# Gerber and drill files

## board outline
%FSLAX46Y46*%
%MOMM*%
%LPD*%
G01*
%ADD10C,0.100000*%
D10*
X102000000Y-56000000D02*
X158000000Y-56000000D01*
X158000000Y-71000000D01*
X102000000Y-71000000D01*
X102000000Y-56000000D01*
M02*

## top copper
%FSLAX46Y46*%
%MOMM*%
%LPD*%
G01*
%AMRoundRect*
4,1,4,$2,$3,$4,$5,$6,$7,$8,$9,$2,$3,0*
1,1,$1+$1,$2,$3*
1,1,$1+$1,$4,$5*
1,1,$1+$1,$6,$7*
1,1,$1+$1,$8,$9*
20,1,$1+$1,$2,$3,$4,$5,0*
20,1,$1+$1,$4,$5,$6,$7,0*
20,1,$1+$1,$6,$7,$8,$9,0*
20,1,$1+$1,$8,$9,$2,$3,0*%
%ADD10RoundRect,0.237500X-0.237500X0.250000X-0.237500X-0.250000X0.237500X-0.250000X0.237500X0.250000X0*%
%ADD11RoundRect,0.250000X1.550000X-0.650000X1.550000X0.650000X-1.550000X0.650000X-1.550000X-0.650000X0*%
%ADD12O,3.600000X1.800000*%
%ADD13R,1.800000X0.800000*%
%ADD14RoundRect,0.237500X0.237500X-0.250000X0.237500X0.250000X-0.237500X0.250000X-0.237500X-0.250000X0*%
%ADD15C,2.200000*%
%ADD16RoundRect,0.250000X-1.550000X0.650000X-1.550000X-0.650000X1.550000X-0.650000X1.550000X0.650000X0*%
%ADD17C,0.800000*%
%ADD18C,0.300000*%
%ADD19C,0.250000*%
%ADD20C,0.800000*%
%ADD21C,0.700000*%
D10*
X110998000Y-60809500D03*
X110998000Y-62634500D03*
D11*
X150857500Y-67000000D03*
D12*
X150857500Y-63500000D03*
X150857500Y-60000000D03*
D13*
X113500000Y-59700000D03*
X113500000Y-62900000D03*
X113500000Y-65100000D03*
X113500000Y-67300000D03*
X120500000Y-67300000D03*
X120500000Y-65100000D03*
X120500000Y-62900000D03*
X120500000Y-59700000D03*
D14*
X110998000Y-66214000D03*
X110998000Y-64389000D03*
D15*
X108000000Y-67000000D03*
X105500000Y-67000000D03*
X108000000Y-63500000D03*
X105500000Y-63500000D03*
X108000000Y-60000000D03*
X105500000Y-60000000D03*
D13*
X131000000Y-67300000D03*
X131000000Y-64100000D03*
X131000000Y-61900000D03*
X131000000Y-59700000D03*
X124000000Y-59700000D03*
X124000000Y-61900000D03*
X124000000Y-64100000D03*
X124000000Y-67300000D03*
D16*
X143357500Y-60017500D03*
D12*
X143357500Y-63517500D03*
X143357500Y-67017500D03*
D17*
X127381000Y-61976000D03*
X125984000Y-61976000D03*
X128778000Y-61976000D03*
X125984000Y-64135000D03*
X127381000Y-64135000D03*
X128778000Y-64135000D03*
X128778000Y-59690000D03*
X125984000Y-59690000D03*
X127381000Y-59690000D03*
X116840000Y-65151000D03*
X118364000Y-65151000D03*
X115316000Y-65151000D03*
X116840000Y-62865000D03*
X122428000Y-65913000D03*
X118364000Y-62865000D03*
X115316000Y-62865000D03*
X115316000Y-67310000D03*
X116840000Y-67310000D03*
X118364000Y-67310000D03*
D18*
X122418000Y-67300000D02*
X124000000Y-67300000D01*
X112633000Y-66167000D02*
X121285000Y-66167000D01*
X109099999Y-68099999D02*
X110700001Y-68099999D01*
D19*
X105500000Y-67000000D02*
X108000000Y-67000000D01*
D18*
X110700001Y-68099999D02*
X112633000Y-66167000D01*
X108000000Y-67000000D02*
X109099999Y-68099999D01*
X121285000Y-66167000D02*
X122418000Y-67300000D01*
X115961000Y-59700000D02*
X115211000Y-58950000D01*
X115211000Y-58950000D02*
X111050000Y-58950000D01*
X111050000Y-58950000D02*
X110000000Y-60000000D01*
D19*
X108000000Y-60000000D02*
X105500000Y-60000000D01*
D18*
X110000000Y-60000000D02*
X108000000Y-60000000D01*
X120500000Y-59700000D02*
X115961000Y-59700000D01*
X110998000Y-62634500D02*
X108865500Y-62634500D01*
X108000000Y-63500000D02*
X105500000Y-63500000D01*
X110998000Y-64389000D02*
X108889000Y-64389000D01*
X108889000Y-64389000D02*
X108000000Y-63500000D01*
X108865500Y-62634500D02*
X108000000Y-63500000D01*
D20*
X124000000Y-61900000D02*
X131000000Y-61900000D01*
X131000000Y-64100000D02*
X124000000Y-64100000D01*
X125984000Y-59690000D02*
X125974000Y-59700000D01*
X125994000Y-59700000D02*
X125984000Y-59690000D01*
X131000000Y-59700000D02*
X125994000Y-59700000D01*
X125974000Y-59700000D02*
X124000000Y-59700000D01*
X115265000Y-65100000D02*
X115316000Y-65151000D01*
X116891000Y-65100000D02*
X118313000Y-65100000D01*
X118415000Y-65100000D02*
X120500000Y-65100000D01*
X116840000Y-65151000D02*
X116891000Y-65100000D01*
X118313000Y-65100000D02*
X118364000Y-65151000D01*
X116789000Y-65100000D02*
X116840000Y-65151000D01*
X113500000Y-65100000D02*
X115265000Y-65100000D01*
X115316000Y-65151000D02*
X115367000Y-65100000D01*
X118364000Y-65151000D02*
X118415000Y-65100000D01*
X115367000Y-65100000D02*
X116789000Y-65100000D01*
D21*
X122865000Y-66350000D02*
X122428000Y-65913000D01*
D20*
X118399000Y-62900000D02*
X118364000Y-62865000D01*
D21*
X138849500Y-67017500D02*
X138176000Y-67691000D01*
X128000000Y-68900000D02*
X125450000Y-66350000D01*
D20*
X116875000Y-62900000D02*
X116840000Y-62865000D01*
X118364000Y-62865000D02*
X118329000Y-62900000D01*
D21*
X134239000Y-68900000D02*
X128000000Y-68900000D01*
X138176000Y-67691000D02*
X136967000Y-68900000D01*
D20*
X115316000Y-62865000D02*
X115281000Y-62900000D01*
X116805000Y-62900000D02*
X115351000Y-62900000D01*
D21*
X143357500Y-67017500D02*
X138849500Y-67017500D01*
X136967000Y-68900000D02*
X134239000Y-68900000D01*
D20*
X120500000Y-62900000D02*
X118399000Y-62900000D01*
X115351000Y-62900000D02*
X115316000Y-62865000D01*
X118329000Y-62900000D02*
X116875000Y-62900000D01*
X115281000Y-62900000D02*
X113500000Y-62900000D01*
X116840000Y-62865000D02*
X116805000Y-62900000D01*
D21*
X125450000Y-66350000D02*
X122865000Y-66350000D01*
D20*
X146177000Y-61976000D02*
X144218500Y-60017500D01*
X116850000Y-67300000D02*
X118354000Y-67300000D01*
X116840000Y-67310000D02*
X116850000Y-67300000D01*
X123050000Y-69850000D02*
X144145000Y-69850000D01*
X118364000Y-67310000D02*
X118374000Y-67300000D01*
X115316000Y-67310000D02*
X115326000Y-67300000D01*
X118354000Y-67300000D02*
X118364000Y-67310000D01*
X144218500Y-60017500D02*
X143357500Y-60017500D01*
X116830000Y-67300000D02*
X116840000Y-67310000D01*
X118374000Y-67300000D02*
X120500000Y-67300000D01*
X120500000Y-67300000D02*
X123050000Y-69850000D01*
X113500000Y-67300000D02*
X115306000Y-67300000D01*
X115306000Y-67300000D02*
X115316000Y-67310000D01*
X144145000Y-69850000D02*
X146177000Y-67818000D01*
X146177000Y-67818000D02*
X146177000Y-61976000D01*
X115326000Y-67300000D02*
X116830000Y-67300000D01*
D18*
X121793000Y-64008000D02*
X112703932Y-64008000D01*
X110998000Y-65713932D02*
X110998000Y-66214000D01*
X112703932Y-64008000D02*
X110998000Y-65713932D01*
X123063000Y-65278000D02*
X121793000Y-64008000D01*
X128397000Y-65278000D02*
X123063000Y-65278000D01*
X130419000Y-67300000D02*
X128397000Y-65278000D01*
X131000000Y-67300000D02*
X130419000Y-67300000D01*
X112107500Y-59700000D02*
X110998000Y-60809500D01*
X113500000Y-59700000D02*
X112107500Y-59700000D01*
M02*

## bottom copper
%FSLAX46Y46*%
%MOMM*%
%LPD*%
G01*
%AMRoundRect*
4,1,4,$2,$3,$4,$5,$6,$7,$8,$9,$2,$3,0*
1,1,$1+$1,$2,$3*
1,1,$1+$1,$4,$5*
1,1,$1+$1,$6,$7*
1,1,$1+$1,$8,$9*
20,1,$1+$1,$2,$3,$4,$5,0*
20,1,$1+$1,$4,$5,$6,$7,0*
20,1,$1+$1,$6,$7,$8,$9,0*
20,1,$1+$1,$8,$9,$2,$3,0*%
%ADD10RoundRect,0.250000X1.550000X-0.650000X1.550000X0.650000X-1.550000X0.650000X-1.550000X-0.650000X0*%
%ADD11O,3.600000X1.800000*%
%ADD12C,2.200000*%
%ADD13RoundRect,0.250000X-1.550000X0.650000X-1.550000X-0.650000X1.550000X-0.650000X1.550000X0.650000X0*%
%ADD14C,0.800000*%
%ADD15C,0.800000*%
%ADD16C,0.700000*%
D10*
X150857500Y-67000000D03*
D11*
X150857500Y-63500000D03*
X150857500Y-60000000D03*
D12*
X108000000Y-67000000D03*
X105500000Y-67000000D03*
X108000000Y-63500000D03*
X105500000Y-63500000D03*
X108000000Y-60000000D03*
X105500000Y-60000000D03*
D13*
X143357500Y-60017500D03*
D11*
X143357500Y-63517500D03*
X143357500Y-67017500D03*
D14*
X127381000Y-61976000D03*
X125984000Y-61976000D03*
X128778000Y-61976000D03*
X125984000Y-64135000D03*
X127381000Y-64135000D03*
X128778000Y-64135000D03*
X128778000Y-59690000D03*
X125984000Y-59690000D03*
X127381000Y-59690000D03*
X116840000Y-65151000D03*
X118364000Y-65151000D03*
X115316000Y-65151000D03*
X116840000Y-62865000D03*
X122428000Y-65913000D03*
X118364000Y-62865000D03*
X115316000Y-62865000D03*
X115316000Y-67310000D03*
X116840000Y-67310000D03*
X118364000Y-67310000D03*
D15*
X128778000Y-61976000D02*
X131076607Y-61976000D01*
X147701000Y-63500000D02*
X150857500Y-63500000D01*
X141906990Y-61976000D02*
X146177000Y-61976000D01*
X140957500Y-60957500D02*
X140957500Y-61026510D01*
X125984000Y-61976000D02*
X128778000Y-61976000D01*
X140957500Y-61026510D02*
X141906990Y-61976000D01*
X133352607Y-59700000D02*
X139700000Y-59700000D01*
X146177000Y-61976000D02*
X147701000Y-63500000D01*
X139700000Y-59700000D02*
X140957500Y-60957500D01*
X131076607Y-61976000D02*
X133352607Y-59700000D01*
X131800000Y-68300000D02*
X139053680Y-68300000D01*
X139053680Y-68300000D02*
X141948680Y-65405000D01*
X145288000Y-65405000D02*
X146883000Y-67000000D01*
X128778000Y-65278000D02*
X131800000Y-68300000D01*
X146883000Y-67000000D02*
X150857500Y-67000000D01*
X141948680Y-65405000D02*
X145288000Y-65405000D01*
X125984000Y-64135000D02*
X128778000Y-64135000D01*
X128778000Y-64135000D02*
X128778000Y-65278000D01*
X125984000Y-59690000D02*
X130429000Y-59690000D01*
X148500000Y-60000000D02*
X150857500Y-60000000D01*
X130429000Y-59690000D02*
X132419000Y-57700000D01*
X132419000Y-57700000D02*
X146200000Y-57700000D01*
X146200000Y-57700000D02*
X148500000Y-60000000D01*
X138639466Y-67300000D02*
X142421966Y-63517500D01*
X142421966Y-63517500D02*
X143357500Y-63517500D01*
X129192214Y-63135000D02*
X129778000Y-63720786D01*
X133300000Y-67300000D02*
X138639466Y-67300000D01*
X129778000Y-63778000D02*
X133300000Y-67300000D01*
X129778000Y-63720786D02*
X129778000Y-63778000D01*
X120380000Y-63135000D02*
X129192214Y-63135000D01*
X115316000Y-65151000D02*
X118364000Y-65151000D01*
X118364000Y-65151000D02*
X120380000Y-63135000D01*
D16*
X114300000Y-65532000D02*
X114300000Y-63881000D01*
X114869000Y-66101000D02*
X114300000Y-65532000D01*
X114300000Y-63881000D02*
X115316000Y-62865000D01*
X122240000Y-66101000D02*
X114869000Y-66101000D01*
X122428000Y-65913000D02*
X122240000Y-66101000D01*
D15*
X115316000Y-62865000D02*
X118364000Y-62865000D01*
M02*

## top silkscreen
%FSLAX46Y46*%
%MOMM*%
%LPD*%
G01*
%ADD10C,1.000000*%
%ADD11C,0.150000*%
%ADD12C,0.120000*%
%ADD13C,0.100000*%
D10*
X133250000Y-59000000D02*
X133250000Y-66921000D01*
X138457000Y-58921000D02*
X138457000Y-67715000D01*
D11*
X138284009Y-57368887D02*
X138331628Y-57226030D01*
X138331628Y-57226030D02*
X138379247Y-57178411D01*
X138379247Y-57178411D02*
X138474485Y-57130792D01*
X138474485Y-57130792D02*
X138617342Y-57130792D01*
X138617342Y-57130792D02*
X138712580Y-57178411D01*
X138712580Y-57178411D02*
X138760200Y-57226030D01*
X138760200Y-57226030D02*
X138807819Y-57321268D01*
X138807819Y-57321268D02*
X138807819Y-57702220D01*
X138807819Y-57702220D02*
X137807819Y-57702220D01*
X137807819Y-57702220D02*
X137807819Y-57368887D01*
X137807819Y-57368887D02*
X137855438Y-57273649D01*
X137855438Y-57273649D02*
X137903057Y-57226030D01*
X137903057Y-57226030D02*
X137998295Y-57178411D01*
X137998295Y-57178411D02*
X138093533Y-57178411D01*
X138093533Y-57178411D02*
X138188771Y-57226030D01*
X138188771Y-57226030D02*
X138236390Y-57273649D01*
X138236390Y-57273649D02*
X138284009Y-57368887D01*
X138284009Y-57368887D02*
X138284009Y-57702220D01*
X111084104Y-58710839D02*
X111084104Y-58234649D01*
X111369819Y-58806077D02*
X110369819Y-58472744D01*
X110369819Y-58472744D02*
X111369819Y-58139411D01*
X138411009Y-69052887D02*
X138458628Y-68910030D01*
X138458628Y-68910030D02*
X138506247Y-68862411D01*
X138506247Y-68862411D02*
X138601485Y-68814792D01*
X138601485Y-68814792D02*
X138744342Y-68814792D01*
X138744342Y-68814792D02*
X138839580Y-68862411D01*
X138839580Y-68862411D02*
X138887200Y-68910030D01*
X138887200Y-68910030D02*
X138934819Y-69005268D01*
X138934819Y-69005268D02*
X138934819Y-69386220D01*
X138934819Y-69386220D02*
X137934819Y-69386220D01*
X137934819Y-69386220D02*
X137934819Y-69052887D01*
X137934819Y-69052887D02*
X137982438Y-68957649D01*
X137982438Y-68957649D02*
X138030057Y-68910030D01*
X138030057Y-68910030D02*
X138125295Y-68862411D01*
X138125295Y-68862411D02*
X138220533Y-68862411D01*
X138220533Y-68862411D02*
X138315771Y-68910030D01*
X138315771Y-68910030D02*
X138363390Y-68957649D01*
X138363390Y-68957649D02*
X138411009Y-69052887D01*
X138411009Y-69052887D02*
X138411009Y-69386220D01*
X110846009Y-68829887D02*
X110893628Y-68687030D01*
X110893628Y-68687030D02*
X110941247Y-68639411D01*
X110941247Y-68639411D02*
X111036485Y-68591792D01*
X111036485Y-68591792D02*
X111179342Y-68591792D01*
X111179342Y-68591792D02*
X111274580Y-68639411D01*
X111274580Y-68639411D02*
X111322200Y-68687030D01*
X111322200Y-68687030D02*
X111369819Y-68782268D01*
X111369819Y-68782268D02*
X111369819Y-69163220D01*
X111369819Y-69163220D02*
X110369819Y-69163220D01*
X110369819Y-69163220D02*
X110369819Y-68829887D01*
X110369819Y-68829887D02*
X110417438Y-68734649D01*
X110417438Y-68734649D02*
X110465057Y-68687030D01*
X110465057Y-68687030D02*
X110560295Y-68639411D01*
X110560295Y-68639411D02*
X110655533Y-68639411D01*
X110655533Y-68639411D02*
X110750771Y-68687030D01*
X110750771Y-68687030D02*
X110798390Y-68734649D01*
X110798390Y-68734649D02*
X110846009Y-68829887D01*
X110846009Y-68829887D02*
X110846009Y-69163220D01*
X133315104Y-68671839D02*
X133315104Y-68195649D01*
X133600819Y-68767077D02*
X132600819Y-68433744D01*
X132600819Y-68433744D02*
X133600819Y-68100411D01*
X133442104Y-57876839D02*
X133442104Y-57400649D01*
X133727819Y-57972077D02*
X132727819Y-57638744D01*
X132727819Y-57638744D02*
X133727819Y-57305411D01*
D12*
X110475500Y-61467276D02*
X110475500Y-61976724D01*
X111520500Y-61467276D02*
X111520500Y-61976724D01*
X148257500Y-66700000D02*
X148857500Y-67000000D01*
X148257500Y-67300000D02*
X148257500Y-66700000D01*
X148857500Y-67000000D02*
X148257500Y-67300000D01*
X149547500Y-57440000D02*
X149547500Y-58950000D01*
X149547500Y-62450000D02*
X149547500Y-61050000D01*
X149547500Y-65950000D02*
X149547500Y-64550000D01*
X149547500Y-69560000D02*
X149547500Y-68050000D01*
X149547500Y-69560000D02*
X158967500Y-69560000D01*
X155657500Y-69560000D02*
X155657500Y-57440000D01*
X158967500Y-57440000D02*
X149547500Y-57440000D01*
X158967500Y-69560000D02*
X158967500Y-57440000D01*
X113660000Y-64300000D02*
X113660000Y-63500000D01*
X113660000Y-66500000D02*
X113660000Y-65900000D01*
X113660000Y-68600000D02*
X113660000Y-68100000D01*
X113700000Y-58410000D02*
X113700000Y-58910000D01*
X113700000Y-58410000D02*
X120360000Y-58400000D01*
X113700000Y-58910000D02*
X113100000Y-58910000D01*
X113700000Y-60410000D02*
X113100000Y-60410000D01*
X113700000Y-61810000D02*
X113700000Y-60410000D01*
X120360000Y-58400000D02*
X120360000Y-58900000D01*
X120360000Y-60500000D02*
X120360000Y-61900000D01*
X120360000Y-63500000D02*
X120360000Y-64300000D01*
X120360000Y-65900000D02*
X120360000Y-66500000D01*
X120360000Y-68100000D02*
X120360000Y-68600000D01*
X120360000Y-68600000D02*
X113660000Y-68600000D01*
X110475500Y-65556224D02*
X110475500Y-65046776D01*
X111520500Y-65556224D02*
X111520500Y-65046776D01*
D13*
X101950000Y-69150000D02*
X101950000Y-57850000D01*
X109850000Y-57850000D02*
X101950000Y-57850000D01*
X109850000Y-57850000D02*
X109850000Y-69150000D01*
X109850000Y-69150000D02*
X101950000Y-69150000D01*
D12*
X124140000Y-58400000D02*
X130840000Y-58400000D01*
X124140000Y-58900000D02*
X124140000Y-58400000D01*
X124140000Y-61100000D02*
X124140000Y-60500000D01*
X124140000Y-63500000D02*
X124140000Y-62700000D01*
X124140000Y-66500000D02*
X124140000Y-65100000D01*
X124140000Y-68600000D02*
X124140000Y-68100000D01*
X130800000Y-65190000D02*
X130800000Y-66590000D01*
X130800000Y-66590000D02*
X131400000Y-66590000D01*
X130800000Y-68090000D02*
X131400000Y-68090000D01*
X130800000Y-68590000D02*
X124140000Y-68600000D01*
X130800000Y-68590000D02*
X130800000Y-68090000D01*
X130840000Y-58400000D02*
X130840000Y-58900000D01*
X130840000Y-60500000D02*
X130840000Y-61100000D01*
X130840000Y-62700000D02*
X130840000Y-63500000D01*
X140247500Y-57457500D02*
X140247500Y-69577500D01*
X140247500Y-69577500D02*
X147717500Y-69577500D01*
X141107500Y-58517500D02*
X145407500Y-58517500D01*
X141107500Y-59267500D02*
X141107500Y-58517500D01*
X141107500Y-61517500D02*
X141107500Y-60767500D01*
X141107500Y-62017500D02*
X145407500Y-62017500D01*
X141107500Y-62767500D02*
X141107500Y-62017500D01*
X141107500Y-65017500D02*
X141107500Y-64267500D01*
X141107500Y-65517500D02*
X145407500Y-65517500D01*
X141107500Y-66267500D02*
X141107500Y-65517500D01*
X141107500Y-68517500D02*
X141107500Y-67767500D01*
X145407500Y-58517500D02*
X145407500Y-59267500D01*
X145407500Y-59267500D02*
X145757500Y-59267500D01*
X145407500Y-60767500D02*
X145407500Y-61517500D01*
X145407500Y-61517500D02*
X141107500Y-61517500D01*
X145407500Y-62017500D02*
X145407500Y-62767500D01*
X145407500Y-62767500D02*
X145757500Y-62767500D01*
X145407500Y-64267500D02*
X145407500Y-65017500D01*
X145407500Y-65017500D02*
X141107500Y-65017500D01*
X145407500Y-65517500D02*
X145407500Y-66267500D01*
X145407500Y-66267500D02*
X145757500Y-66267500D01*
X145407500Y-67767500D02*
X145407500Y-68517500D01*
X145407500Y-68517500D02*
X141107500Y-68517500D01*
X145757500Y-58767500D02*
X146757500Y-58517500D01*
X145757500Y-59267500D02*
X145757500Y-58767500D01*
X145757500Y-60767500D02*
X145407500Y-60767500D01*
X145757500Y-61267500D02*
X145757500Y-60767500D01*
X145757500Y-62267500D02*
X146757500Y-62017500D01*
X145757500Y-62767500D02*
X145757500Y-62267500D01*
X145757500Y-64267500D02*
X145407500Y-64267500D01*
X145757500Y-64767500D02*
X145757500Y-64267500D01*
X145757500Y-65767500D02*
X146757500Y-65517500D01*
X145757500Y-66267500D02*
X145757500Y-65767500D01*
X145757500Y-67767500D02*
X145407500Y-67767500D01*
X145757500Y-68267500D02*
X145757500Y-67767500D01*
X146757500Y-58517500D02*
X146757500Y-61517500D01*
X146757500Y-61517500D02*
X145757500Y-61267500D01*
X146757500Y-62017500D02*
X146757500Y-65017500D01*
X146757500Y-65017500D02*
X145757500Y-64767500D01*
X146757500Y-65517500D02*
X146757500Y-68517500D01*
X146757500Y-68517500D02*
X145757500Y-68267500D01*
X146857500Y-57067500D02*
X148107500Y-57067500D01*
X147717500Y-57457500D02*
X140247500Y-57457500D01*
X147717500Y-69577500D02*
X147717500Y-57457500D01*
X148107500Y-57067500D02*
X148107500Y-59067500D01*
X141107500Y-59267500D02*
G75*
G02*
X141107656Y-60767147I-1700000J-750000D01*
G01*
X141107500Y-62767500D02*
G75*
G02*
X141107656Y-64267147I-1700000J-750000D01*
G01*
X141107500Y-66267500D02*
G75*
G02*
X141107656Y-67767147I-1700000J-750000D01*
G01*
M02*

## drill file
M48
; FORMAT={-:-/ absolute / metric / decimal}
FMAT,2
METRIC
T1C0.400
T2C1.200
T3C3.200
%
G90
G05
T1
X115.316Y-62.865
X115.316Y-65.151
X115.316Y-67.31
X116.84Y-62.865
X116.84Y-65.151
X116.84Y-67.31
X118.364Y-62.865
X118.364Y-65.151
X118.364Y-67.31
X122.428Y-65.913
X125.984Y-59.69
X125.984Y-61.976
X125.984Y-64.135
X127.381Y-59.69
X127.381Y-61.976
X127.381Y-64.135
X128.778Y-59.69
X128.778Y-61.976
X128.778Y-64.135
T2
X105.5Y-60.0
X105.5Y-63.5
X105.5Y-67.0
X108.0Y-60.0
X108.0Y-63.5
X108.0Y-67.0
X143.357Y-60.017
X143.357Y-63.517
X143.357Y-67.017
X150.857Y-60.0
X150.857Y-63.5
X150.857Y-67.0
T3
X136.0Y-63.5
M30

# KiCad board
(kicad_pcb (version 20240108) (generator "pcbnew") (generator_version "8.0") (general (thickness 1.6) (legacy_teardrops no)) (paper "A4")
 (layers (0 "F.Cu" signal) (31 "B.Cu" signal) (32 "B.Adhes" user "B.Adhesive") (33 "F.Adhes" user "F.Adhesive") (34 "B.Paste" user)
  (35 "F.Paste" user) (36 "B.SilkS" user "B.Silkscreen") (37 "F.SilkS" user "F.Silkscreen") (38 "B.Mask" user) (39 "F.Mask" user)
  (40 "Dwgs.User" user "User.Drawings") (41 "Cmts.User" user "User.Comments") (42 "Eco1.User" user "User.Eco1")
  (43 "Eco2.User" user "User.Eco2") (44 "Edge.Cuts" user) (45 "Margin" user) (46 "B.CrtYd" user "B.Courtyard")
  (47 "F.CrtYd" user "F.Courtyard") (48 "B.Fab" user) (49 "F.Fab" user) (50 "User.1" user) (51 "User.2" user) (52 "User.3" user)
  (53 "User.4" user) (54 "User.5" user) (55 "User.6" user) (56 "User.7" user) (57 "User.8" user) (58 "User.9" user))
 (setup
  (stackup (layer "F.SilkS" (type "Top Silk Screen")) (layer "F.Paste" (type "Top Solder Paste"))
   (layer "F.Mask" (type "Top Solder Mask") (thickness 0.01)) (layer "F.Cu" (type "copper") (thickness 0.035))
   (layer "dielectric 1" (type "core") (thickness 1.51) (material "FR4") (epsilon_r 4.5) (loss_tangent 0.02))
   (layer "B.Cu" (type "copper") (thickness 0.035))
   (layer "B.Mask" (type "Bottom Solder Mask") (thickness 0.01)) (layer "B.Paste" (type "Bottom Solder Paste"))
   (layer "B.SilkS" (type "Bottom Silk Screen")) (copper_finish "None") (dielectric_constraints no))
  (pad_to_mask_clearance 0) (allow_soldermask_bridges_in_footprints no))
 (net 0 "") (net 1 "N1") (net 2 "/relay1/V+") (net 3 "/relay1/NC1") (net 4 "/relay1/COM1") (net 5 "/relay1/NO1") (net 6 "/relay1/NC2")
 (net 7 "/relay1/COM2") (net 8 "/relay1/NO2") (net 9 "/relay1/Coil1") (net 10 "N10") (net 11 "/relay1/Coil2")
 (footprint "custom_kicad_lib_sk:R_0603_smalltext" (layer "F.Cu") (at 110.998 61.722 -90)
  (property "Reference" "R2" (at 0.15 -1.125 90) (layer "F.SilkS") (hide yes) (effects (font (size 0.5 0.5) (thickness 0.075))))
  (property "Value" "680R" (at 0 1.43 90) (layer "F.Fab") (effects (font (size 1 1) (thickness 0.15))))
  (fp_line (start -0.254724 0.5225) (end 0.254724 0.5225) (stroke (width 0.12) (type solid)) (layer "F.SilkS"))
  (fp_line (start -0.254724 -0.5225) (end 0.254724 -0.5225) (stroke (width 0.12) (type solid)) (layer "F.SilkS"))
  (pad "1" smd roundrect (at -0.9125 0 270) (size 0.975 0.95) (layers "F.Cu" "F.Paste" "F.Mask") (roundrect_rratio 0.25) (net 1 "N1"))
  (pad "2" smd roundrect (at 0.9125 0 270) (size 0.975 0.95) (layers "F.Cu" "F.Paste" "F.Mask") (roundrect_rratio 0.25) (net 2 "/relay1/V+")))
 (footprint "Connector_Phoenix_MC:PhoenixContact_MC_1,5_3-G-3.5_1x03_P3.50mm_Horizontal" (layer "F.Cu") (at 150.8575 67 90)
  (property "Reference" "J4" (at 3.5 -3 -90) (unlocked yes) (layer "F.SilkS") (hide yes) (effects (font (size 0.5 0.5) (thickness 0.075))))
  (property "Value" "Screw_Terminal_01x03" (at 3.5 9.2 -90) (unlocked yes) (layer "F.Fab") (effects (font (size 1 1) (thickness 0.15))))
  (fp_line (start 0.3 -2.6) (end 0 -2) (stroke (width 0.12) (type solid)) (layer "F.SilkS"))
  (fp_line (start -0.3 -2.6) (end 0.3 -2.6) (stroke (width 0.12) (type solid)) (layer "F.SilkS"))
  (fp_line (start 0 -2) (end -0.3 -2.6) (stroke (width 0.12) (type solid)) (layer "F.SilkS"))
  (fp_line (start 9.56 -1.31) (end 8.05 -1.31) (stroke (width 0.12) (type solid)) (layer "F.SilkS"))
  (fp_line (start 4.55 -1.31) (end 5.95 -1.31) (stroke (width 0.12) (type solid)) (layer "F.SilkS"))
  (fp_line (start 1.05 -1.31) (end 2.45 -1.31) (stroke (width 0.12) (type solid)) (layer "F.SilkS"))
  (fp_line (start -2.56 -1.31) (end -1.05 -1.31) (stroke (width 0.12) (type solid)) (layer "F.SilkS"))
  (fp_line (start -2.56 -1.31) (end -2.56 8.11) (stroke (width 0.12) (type solid)) (layer "F.SilkS"))
  (fp_line (start -2.56 4.8) (end 9.56 4.8) (stroke (width 0.12) (type solid)) (layer "F.SilkS"))
  (fp_line (start 9.56 8.11) (end 9.56 -1.31) (stroke (width 0.12) (type solid)) (layer "F.SilkS"))
  (fp_line (start -2.56 8.11) (end 9.56 8.11) (stroke (width 0.12) (type solid)) (layer "F.SilkS"))
  (pad "1" thru_hole roundrect (at 0 0 90) (size 1.8 3.6) (drill 1.2) (layers "*.Cu" "*.Mask") (remove_unused_layers no)
   (roundrect_rratio 0.138889) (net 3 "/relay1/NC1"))
  (pad "2" thru_hole oval (at 3.5 0 90) (size 1.8 3.6) (drill 1.2) (layers "*.Cu" "*.Mask") (remove_unused_layers no) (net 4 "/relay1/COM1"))
  (pad "3" thru_hole oval (at 7 0 90) (size 1.8 3.6) (drill 1.2) (layers "*.Cu" "*.Mask") (remove_unused_layers no) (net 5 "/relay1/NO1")))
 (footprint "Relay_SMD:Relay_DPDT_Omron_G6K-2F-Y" (layer "F.Cu") (at 117 63.5)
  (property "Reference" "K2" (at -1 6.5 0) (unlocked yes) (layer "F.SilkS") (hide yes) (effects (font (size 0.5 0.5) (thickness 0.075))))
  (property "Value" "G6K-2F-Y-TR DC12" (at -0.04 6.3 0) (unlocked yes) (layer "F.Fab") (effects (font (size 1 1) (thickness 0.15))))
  (fp_line (start -3.34 0.8) (end -3.34 0) (stroke (width 0.12) (type solid)) (layer "F.SilkS"))
  (fp_line (start -3.34 3) (end -3.34 2.4) (stroke (width 0.12) (type solid)) (layer "F.SilkS"))
  (fp_line (start -3.34 5.1) (end -3.34 4.6) (stroke (width 0.12) (type solid)) (layer "F.SilkS"))
  (fp_line (start -3.3 -5.09) (end -3.3 -4.59) (stroke (width 0.12) (type solid)) (layer "F.SilkS"))
  (fp_line (start -3.3 -5.09) (end 3.36 -5.1) (stroke (width 0.12) (type solid)) (layer "F.SilkS"))
  (fp_line (start -3.3 -4.59) (end -3.9 -4.59) (stroke (width 0.12) (type solid)) (layer "F.SilkS"))
  (fp_line (start -3.3 -3.09) (end -3.9 -3.09) (stroke (width 0.12) (type solid)) (layer "F.SilkS"))
  (fp_line (start -3.3 -1.69) (end -3.3 -3.09) (stroke (width 0.12) (type solid)) (layer "F.SilkS"))
  (fp_line (start 3.36 -5.1) (end 3.36 -4.6) (stroke (width 0.12) (type solid)) (layer "F.SilkS"))
  (fp_line (start 3.36 -3) (end 3.36 -1.6) (stroke (width 0.12) (type solid)) (layer "F.SilkS"))
  (fp_line (start 3.36 0) (end 3.36 0.8) (stroke (width 0.12) (type solid)) (layer "F.SilkS"))
  (fp_line (start 3.36 2.4) (end 3.36 3) (stroke (width 0.12) (type solid)) (layer "F.SilkS"))
  (fp_line (start 3.36 4.6) (end 3.36 5.1) (stroke (width 0.12) (type solid)) (layer "F.SilkS"))
  (fp_line (start 3.36 5.1) (end -3.34 5.1) (stroke (width 0.12) (type solid)) (layer "F.SilkS"))
  (pad "1" smd rect (at -3.5 -3.8) (size 1.8 0.8) (layers "F.Cu" "F.Paste" "F.Mask") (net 1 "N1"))
  (pad "2" smd rect (at -3.5 -0.6) (size 1.8 0.8) (layers "F.Cu" "F.Paste" "F.Mask") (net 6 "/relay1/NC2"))
  (pad "3" smd rect (at -3.5 1.6) (size 1.8 0.8) (layers "F.Cu" "F.Paste" "F.Mask") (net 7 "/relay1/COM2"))
  (pad "4" smd rect (at -3.5 3.8) (size 1.8 0.8) (layers "F.Cu" "F.Paste" "F.Mask") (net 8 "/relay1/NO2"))
  (pad "5" smd rect (at 3.5 3.8) (size 1.8 0.8) (layers "F.Cu" "F.Paste" "F.Mask") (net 8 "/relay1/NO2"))
  (pad "6" smd rect (at 3.5 1.6) (size 1.8 0.8) (layers "F.Cu" "F.Paste" "F.Mask") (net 7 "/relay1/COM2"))
  (pad "7" smd rect (at 3.5 -0.6) (size 1.8 0.8) (layers "F.Cu" "F.Paste" "F.Mask") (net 6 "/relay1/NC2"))
  (pad "8" smd rect (at 3.5 -3.8) (size 1.8 0.8) (layers "F.Cu" "F.Paste" "F.Mask") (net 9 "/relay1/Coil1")))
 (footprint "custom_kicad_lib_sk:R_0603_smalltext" (layer "F.Cu") (at 110.998 65.3015 90)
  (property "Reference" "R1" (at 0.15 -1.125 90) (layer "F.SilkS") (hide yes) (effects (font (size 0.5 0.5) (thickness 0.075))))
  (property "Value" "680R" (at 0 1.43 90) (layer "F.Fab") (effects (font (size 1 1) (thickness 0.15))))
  (fp_line (start -0.254724 -0.5225) (end 0.254724 -0.5225) (stroke (width 0.12) (type solid)) (layer "F.SilkS"))
  (fp_line (start -0.254724 0.5225) (end 0.254724 0.5225) (stroke (width 0.12) (type solid)) (layer "F.SilkS"))
  (pad "1" smd roundrect (at -0.9125 0 90) (size 0.975 0.95) (layers "F.Cu" "F.Paste" "F.Mask") (roundrect_rratio 0.25) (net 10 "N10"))
  (pad "2" smd roundrect (at 0.9125 0 90) (size 0.975 0.95) (layers "F.Cu" "F.Paste" "F.Mask") (roundrect_rratio 0.25) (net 2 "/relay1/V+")))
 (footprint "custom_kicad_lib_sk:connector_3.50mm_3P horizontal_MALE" (layer "F.Cu") (at 108 63.5 -90)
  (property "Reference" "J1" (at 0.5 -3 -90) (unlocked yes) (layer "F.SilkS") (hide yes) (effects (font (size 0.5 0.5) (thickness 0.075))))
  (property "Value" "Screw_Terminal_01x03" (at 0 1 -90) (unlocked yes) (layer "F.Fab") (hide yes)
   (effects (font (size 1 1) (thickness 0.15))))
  (fp_line (start 5.65 6.05) (end -5.65 6.05) (stroke (width 0.1) (type default)) (layer "F.SilkS"))
  (fp_line (start -5.65 -1.85) (end -5.65 6.05) (stroke (width 0.1) (type default)) (layer "F.SilkS"))
  (fp_line (start -5.65 -1.85) (end 5.65 -1.85) (stroke (width 0.1) (type default)) (layer "F.SilkS"))
  (fp_line (start 5.65 -1.85) (end 5.65 6.05) (stroke (width 0.1) (type default)) (layer "F.SilkS"))
  (pad "1" thru_hole circle (at 3.5 0 270) (size 2.2 2.2) (drill 1.2) (layers "*.Cu" "*.Mask") (remove_unused_layers no)
   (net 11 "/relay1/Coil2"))
  (pad "1" thru_hole circle (at 3.5 2.5 270) (size 2.2 2.2) (drill 1.2) (layers "*.Cu" "*.Mask") (remove_unused_layers no)
   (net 11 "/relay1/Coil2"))
  (pad "2" thru_hole circle (at 0 0 270) (size 2.2 2.2) (drill 1.2) (layers "*.Cu" "*.Mask") (remove_unused_layers no) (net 2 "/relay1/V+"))
  (pad "2" thru_hole circle (at 0 2.5 270) (size 2.2 2.2) (drill 1.2) (layers "*.Cu" "*.Mask") (remove_unused_layers no)
   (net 2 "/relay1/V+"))
  (pad "3" thru_hole circle (at -3.5 0 270) (size 2.2 2.2) (drill 1.2) (layers "*.Cu" "*.Mask") (remove_unused_layers no)
   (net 9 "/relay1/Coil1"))
  (pad "3" thru_hole circle (at -3.5 2.5 270) (size 2.2 2.2) (drill 1.2) (layers "*.Cu" "*.Mask") (remove_unused_layers no)
   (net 9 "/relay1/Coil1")))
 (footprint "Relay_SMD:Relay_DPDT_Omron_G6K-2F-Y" (layer "F.Cu") (at 127.5 63.5 180)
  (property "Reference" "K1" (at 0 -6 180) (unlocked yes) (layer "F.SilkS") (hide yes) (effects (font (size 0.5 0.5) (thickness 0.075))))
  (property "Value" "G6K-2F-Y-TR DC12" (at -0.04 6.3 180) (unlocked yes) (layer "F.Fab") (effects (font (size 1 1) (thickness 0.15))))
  (fp_line (start 3.36 5.1) (end -3.34 5.1) (stroke (width 0.12) (type solid)) (layer "F.SilkS"))
  (fp_line (start 3.36 4.6) (end 3.36 5.1) (stroke (width 0.12) (type solid)) (layer "F.SilkS"))
  (fp_line (start 3.36 2.4) (end 3.36 3) (stroke (width 0.12) (type solid)) (layer "F.SilkS"))
  (fp_line (start 3.36 0) (end 3.36 0.8) (stroke (width 0.12) (type solid)) (layer "F.SilkS"))
  (fp_line (start 3.36 -3) (end 3.36 -1.6) (stroke (width 0.12) (type solid)) (layer "F.SilkS"))
  (fp_line (start 3.36 -5.1) (end 3.36 -4.6) (stroke (width 0.12) (type solid)) (layer "F.SilkS"))
  (fp_line (start -3.3 -1.69) (end -3.3 -3.09) (stroke (width 0.12) (type solid)) (layer "F.SilkS"))
  (fp_line (start -3.3 -3.09) (end -3.9 -3.09) (stroke (width 0.12) (type solid)) (layer "F.SilkS"))
  (fp_line (start -3.3 -4.59) (end -3.9 -4.59) (stroke (width 0.12) (type solid)) (layer "F.SilkS"))
  (fp_line (start -3.3 -5.09) (end 3.36 -5.1) (stroke (width 0.12) (type solid)) (layer "F.SilkS"))
  (fp_line (start -3.3 -5.09) (end -3.3 -4.59) (stroke (width 0.12) (type solid)) (layer "F.SilkS"))
  (fp_line (start -3.34 5.1) (end -3.34 4.6) (stroke (width 0.12) (type solid)) (layer "F.SilkS"))
  (fp_line (start -3.34 3) (end -3.34 2.4) (stroke (width 0.12) (type solid)) (layer "F.SilkS"))
  (fp_line (start -3.34 0.8) (end -3.34 0) (stroke (width 0.12) (type solid)) (layer "F.SilkS"))
  (pad "1" smd rect (at -3.5 -3.8 180) (size 1.8 0.8) (layers "F.Cu" "F.Paste" "F.Mask") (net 10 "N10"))
  (pad "2" smd rect (at -3.5 -0.6 180) (size 1.8 0.8) (layers "F.Cu" "F.Paste" "F.Mask") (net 3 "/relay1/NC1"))
  (pad "3" smd rect (at -3.5 1.6 180) (size 1.8 0.8) (layers "F.Cu" "F.Paste" "F.Mask") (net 4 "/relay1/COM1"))
  (pad "4" smd rect (at -3.5 3.8 180) (size 1.8 0.8) (layers "F.Cu" "F.Paste" "F.Mask") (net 5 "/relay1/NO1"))
  (pad "5" smd rect (at 3.5 3.8 180) (size 1.8 0.8) (layers "F.Cu" "F.Paste" "F.Mask") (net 5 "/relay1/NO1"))
  (pad "6" smd rect (at 3.5 1.6 180) (size 1.8 0.8) (layers "F.Cu" "F.Paste" "F.Mask") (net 4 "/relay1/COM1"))
  (pad "7" smd rect (at 3.5 -0.6 180) (size 1.8 0.8) (layers "F.Cu" "F.Paste" "F.Mask") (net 3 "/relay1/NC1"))
  (pad "8" smd rect (at 3.5 -3.8 180) (size 1.8 0.8) (layers "F.Cu" "F.Paste" "F.Mask") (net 11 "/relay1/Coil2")))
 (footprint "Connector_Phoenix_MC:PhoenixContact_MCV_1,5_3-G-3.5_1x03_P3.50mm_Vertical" (layer "F.Cu") (at 143.3575 60.0175 -90)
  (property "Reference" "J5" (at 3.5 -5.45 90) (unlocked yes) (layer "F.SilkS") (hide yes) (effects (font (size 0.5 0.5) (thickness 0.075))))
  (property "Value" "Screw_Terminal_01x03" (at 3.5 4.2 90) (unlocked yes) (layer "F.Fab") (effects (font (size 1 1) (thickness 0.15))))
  (fp_line (start -2.56 3.11) (end 9.56 3.11) (stroke (width 0.12) (type solid)) (layer "F.SilkS"))
  (fp_line (start 9.56 3.11) (end 9.56 -4.36) (stroke (width 0.12) (type solid)) (layer "F.SilkS"))
  (fp_line (start -1.5 2.25) (end -1.5 -2.05) (stroke (width 0.12) (type solid)) (layer "F.SilkS"))
  (fp_line (start -0.75 2.25) (end -1.5 2.25) (stroke (width 0.12) (type solid)) (layer "F.SilkS"))
  (fp_line (start 1.5 2.25) (end 0.75 2.25) (stroke (width 0.12) (type solid)) (layer "F.SilkS"))
  (fp_line (start 2 2.25) (end 2 -2.05) (stroke (width 0.12) (type solid)) (layer "F.SilkS"))
  (fp_line (start 2.75 2.25) (end 2 2.25) (stroke (width 0.12) (type solid)) (layer "F.SilkS"))
  (fp_line (start 5 2.25) (end 4.25 2.25) (stroke (width 0.12) (type solid)) (layer "F.SilkS"))
  (fp_line (start 5.5 2.25) (end 5.5 -2.05) (stroke (width 0.12) (type solid)) (layer "F.SilkS"))
  (fp_line (start 6.25 2.25) (end 5.5 2.25) (stroke (width 0.12) (type solid)) (layer "F.SilkS"))
  (fp_line (start 8.5 2.25) (end 7.75 2.25) (stroke (width 0.12) (type solid)) (layer "F.SilkS"))
  (fp_line (start -1.5 -2.05) (end -0.75 -2.05) (stroke (width 0.12) (type solid)) (layer "F.SilkS"))
  (fp_line (start -0.75 -2.05) (end -0.75 -2.4) (stroke (width 0.12) (type solid)) (layer "F.SilkS"))
  (fp_line (start 0.75 -2.05) (end 1.5 -2.05) (stroke (width 0.12) (type solid)) (layer "F.SilkS"))
  (fp_line (start 1.5 -2.05) (end 1.5 2.25) (stroke (width 0.12) (type solid)) (layer "F.SilkS"))
  (fp_line (start 2 -2.05) (end 2.75 -2.05) (stroke (width 0.12) (type solid)) (layer "F.SilkS"))
  (fp_line (start 2.75 -2.05) (end 2.75 -2.4) (stroke (width 0.12) (type solid)) (layer "F.SilkS"))
  (fp_line (start 4.25 -2.05) (end 5 -2.05) (stroke (width 0.12) (type solid)) (layer "F.SilkS"))
  (fp_line (start 5 -2.05) (end 5 2.25) (stroke (width 0.12) (type solid)) (layer "F.SilkS"))
  (fp_line (start 5.5 -2.05) (end 6.25 -2.05) (stroke (width 0.12) (type solid)) (layer "F.SilkS"))
  (fp_line (start 6.25 -2.05) (end 6.25 -2.4) (stroke (width 0.12) (type solid)) (layer "F.SilkS"))
  (fp_line (start 7.75 -2.05) (end 8.5 -2.05) (stroke (width 0.12) (type solid)) (layer "F.SilkS"))
  (fp_line (start 8.5 -2.05) (end 8.5 2.25) (stroke (width 0.12) (type solid)) (layer "F.SilkS"))
  (fp_line (start -1.25 -2.4) (end -1.5 -3.4) (stroke (width 0.12) (type solid)) (layer "F.SilkS"))
  (fp_line (start -0.75 -2.4) (end -1.25 -2.4) (stroke (width 0.12) (type solid)) (layer "F.SilkS"))
  (fp_line (start 0.75 -2.4) (end 0.75 -2.05) (stroke (width 0.12) (type solid)) (layer "F.SilkS"))
  (fp_line (start 1.25 -2.4) (end 0.75 -2.4) (stroke (width 0.12) (type solid)) (layer "F.SilkS"))
  (fp_line (start 2.25 -2.4) (end 2 -3.4) (stroke (width 0.12) (type solid)) (layer "F.SilkS"))
  (fp_line (start 2.75 -2.4) (end 2.25 -2.4) (stroke (width 0.12) (type solid)) (layer "F.SilkS"))
  (fp_line (start 4.25 -2.4) (end 4.25 -2.05) (stroke (width 0.12) (type solid)) (layer "F.SilkS"))
  (fp_line (start 4.75 -2.4) (end 4.25 -2.4) (stroke (width 0.12) (type solid)) (layer "F.SilkS"))
  (fp_line (start 5.75 -2.4) (end 5.5 -3.4) (stroke (width 0.12) (type solid)) (layer "F.SilkS"))
  (fp_line (start 6.25 -2.4) (end 5.75 -2.4) (stroke (width 0.12) (type solid)) (layer "F.SilkS"))
  (fp_line (start 7.75 -2.4) (end 7.75 -2.05) (stroke (width 0.12) (type solid)) (layer "F.SilkS"))
  (fp_line (start 8.25 -2.4) (end 7.75 -2.4) (stroke (width 0.12) (type solid)) (layer "F.SilkS"))
  (fp_line (start -1.5 -3.4) (end 1.5 -3.4) (stroke (width 0.12) (type solid)) (layer "F.SilkS"))
  (fp_line (start 1.5 -3.4) (end 1.25 -2.4) (stroke (width 0.12) (type solid)) (layer "F.SilkS"))
  (fp_line (start 2 -3.4) (end 5 -3.4) (stroke (width 0.12) (type solid)) (layer "F.SilkS"))
  (fp_line (start 5 -3.4) (end 4.75 -2.4) (stroke (width 0.12) (type solid)) (layer "F.SilkS"))
  (fp_line (start 5.5 -3.4) (end 8.5 -3.4) (stroke (width 0.12) (type solid)) (layer "F.SilkS"))
  (fp_line (start 8.5 -3.4) (end 8.25 -2.4) (stroke (width 0.12) (type solid)) (layer "F.SilkS"))
  (fp_line (start -2.95 -3.5) (end -2.95 -4.75) (stroke (width 0.12) (type solid)) (layer "F.SilkS"))
  (fp_line (start -2.56 -4.36) (end -2.56 3.11) (stroke (width 0.12) (type solid)) (layer "F.SilkS"))
  (fp_line (start 9.56 -4.36) (end -2.56 -4.36) (stroke (width 0.12) (type solid)) (layer "F.SilkS"))
  (fp_line (start -2.95 -4.75) (end -0.95 -4.75) (stroke (width 0.12) (type solid)) (layer "F.SilkS"))
  (fp_arc (start -0.75 2.25) (mid -0.000193 2.09191) (end 0.749647 2.249844) (stroke (width 0.12) (type solid)) (layer "F.SilkS"))
  (fp_arc (start 2.75 2.25) (mid 3.499807 2.09191) (end 4.249647 2.249844) (stroke (width 0.12) (type solid)) (layer "F.SilkS"))
  (fp_arc (start 6.25 2.25) (mid 6.999807 2.09191) (end 7.749647 2.249844) (stroke (width 0.12) (type solid)) (layer "F.SilkS"))
  (pad "1" thru_hole roundrect (at 0 0 270) (size 1.8 3.6) (drill 1.2) (layers "*.Cu" "*.Mask") (remove_unused_layers no)
   (roundrect_rratio 0.138889) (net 8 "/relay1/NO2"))
  (pad "2" thru_hole oval (at 3.5 0 270) (size 1.8 3.6) (drill 1.2) (layers "*.Cu" "*.Mask") (remove_unused_layers no)
   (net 7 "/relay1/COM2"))
  (pad "3" thru_hole oval (at 7 0 270) (size 1.8 3.6) (drill 1.2) (layers "*.Cu" "*.Mask") (remove_unused_layers no) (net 6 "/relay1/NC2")))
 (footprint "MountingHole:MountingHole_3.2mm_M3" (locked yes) (layer "F.Cu") (at 136 63.5)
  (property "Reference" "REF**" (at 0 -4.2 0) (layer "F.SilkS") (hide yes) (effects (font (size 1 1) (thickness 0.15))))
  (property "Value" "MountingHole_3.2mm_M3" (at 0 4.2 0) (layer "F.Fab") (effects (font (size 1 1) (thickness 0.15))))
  (pad "" np_thru_hole circle (at 0 0) (size 3.2 3.2) (drill 3.2) (layers "*.Cu" "*.Mask")))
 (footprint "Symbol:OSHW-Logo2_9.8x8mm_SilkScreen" (layer "B.Cu") (at 120.396 63.627 -90)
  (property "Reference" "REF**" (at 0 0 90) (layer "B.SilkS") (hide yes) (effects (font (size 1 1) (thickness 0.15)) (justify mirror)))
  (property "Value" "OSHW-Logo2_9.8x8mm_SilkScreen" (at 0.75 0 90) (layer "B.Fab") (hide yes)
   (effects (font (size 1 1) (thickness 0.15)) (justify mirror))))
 (gr_line (start 133.25 59) (end 133.25 66.921) (stroke (width 1) (type default)) (layer "F.SilkS"))
 (gr_line (start 138.457 58.921) (end 138.457 67.715) (stroke (width 1) (type default)) (layer "F.SilkS"))
 (gr_rect (start 102 56) (end 158 71) (stroke (width 0.1) (type default)) (fill none) (layer "Edge.Cuts"))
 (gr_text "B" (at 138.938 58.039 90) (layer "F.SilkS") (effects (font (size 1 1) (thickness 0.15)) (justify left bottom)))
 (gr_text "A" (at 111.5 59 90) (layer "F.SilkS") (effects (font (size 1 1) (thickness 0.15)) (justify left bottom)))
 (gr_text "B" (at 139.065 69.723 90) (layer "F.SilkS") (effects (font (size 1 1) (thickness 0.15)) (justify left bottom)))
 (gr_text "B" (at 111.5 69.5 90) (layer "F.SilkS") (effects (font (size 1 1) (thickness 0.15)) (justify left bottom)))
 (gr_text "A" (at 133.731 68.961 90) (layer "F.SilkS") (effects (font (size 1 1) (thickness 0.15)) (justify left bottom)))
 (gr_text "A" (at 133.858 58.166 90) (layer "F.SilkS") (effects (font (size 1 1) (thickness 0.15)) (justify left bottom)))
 (segment (start 122.418 67.3) (end 124 67.3) (width 0.3) (layer "F.Cu") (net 11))
 (segment (start 112.633 66.167) (end 121.285 66.167) (width 0.3) (layer "F.Cu") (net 11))
 (segment (start 109.099999 68.099999) (end 110.700001 68.099999) (width 0.3) (layer "F.Cu") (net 11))
 (segment (start 105.5 67) (end 108 67) (width 0.25) (layer "F.Cu") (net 11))
 (segment (start 110.700001 68.099999) (end 112.633 66.167) (width 0.3) (layer "F.Cu") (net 11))
 (segment (start 108 67) (end 109.099999 68.099999) (width 0.3) (layer "F.Cu") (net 11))
 (segment (start 121.285 66.167) (end 122.418 67.3) (width 0.3) (layer "F.Cu") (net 11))
 (segment (start 115.961 59.7) (end 115.211 58.95) (width 0.3) (layer "F.Cu") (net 9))
 (segment (start 115.211 58.95) (end 111.05 58.95) (width 0.3) (layer "F.Cu") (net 9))
 (segment (start 111.05 58.95) (end 110 60) (width 0.3) (layer "F.Cu") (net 9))
 (segment (start 108 60) (end 105.5 60) (width 0.25) (layer "F.Cu") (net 9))
 (segment (start 110 60) (end 108 60) (width 0.3) (layer "F.Cu") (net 9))
 (segment (start 120.5 59.7) (end 115.961 59.7) (width 0.3) (layer "F.Cu") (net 9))
 (segment (start 110.998 62.6345) (end 108.8655 62.6345) (width 0.3) (layer "F.Cu") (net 2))
 (segment (start 108 63.5) (end 105.5 63.5) (width 0.3) (layer "F.Cu") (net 2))
 (segment (start 110.998 64.389) (end 108.889 64.389) (width 0.3) (layer "F.Cu") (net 2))
 (segment (start 108.889 64.389) (end 108 63.5) (width 0.3) (layer "F.Cu") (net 2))
 (segment (start 108.8655 62.6345) (end 108 63.5) (width 0.3) (layer "F.Cu") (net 2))
 (segment (start 124 61.9) (end 131 61.9) (width 0.8) (layer "F.Cu") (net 4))
 (via (at 127.381 61.976) (size 0.8) (drill 0.4) (layers "F.Cu" "B.Cu") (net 4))
 (via (at 125.984 61.976) (size 0.8) (drill 0.4) (layers "F.Cu" "B.Cu") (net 4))
 (via (at 128.778 61.976) (size 0.8) (drill 0.4) (layers "F.Cu" "B.Cu") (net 4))
 (segment (start 128.778 61.976) (end 131.076607 61.976) (width 0.8) (layer "B.Cu") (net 4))
 (segment (start 147.701 63.5) (end 150.8575 63.5) (width 0.8) (layer "B.Cu") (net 4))
 (segment (start 141.90699 61.976) (end 146.177 61.976) (width 0.8) (layer "B.Cu") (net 4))
 (segment (start 140.9575 60.9575) (end 140.9575 61.02651) (width 0.8) (layer "B.Cu") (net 4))
 (segment (start 125.984 61.976) (end 128.778 61.976) (width 0.8) (layer "B.Cu") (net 4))
 (segment (start 140.9575 61.02651) (end 141.90699 61.976) (width 0.8) (layer "B.Cu") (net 4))
 (segment (start 133.352607 59.7) (end 139.7 59.7) (width 0.8) (layer "B.Cu") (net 4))
 (segment (start 146.177 61.976) (end 147.701 63.5) (width 0.8) (layer "B.Cu") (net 4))
 (segment (start 139.7 59.7) (end 140.9575 60.9575) (width 0.8) (layer "B.Cu") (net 4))
 (segment (start 131.076607 61.976) (end 133.352607 59.7) (width 0.8) (layer "B.Cu") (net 4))
 (segment (start 131 64.1) (end 124 64.1) (width 0.8) (layer "F.Cu") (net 3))
 (via (at 125.984 64.135) (size 0.8) (drill 0.4) (layers "F.Cu" "B.Cu") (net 3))
 (via (at 127.381 64.135) (size 0.8) (drill 0.4) (layers "F.Cu" "B.Cu") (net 3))
 (via (at 128.778 64.135) (size 0.8) (drill 0.4) (layers "F.Cu" "B.Cu") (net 3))
 (segment (start 131.8 68.3) (end 139.05368 68.3) (width 0.8) (layer "B.Cu") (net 3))
 (segment (start 139.05368 68.3) (end 141.94868 65.405) (width 0.8) (layer "B.Cu") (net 3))
 (segment (start 145.288 65.405) (end 146.883 67) (width 0.8) (layer "B.Cu") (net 3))
 (segment (start 128.778 65.278) (end 131.8 68.3) (width 0.8) (layer "B.Cu") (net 3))
 (segment (start 146.883 67) (end 150.8575 67) (width 0.8) (layer "B.Cu") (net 3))
 (segment (start 141.94868 65.405) (end 145.288 65.405) (width 0.8) (layer "B.Cu") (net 3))
 (segment (start 125.984 64.135) (end 128.778 64.135) (width 0.8) (layer "B.Cu") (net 3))
 (segment (start 128.778 64.135) (end 128.778 65.278) (width 0.8) (layer "B.Cu") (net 3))
 (segment (start 125.984 59.69) (end 125.974 59.7) (width 0.8) (layer "F.Cu") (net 5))
 (segment (start 125.994 59.7) (end 125.984 59.69) (width 0.8) (layer "F.Cu") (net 5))
 (segment (start 131 59.7) (end 125.994 59.7) (width 0.8) (layer "F.Cu") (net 5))
 (segment (start 125.974 59.7) (end 124 59.7) (width 0.8) (layer "F.Cu") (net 5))
 (via (at 128.778 59.69) (size 0.8) (drill 0.4) (layers "F.Cu" "B.Cu") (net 5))
 (via (at 125.984 59.69) (size 0.8) (drill 0.4) (layers "F.Cu" "B.Cu") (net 5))
 (via (at 127.381 59.69) (size 0.8) (drill 0.4) (layers "F.Cu" "B.Cu") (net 5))
 (segment (start 125.984 59.69) (end 130.429 59.69) (width 0.8) (layer "B.Cu") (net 5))
 (segment (start 148.5 60) (end 150.8575 60) (width 0.8) (layer "B.Cu") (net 5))
 (segment (start 130.429 59.69) (end 132.419 57.7) (width 0.8) (layer "B.Cu") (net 5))
 (segment (start 132.419 57.7) (end 146.2 57.7) (width 0.8) (layer "B.Cu") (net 5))
 (segment (start 146.2 57.7) (end 148.5 60) (width 0.8) (layer "B.Cu") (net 5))
 (segment (start 115.265 65.1) (end 115.316 65.151) (width 0.8) (layer "F.Cu") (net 7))
 (segment (start 116.891 65.1) (end 118.313 65.1) (width 0.8) (layer "F.Cu") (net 7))
 (segment (start 118.415 65.1) (end 120.5 65.1) (width 0.8) (layer "F.Cu") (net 7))
 (segment (start 116.84 65.151) (end 116.891 65.1) (width 0.8) (layer "F.Cu") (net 7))
 (segment (start 118.313 65.1) (end 118.364 65.151) (width 0.8) (layer "F.Cu") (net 7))
 (segment (start 116.789 65.1) (end 116.84 65.151) (width 0.8) (layer "F.Cu") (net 7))
 (segment (start 113.5 65.1) (end 115.265 65.1) (width 0.8) (layer "F.Cu") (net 7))
 (segment (start 115.316 65.151) (end 115.367 65.1) (width 0.8) (layer "F.Cu") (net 7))
 (segment (start 118.364 65.151) (end 118.415 65.1) (width 0.8) (layer "F.Cu") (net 7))
 (segment (start 115.367 65.1) (end 116.789 65.1) (width 0.8) (layer "F.Cu") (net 7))
 (via (at 116.84 65.151) (size 0.8) (drill 0.4) (layers "F.Cu" "B.Cu") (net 7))
 (via (at 118.364 65.151) (size 0.8) (drill 0.4) (layers "F.Cu" "B.Cu") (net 7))
 (via (at 115.316 65.151) (size 0.8) (drill 0.4) (layers "F.Cu" "B.Cu") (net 7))
 (segment (start 138.639466 67.3) (end 142.421966 63.5175) (width 0.8) (layer "B.Cu") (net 7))
 (segment (start 142.421966 63.5175) (end 143.3575 63.5175) (width 0.8) (layer "B.Cu") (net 7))
 (segment (start 129.192214 63.135) (end 129.778 63.720786) (width 0.8) (layer "B.Cu") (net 7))
 (segment (start 133.3 67.3) (end 138.639466 67.3) (width 0.8) (layer "B.Cu") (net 7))
 (segment (start 129.778 63.778) (end 133.3 67.3) (width 0.8) (layer "B.Cu") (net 7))
 (segment (start 129.778 63.720786) (end 129.778 63.778) (width 0.8) (layer "B.Cu") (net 7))
 (segment (start 120.38 63.135) (end 129.192214 63.135) (width 0.8) (layer "B.Cu") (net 7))
 (segment (start 115.316 65.151) (end 118.364 65.151) (width 0.8) (layer "B.Cu") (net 7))
 (segment (start 118.364 65.151) (end 120.38 63.135) (width 0.8) (layer "B.Cu") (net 7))
 (segment (start 122.865 66.35) (end 122.428 65.913) (width 0.7) (layer "F.Cu") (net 6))
 (segment (start 118.399 62.9) (end 118.364 62.865) (width 0.8) (layer "F.Cu") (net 6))
 (segment (start 138.8495 67.0175) (end 138.176 67.691) (width 0.7) (layer "F.Cu") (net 6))
 (segment (start 128 68.9) (end 125.45 66.35) (width 0.7) (layer "F.Cu") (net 6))
 (segment (start 116.875 62.9) (end 116.84 62.865) (width 0.8) (layer "F.Cu") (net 6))
 (segment (start 118.364 62.865) (end 118.329 62.9) (width 0.8) (layer "F.Cu") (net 6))
 (segment (start 134.239 68.9) (end 128 68.9) (width 0.7) (layer "F.Cu") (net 6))
 (segment (start 138.176 67.691) (end 136.967 68.9) (width 0.7) (layer "F.Cu") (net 6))
 (segment (start 115.316 62.865) (end 115.281 62.9) (width 0.8) (layer "F.Cu") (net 6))
 (segment (start 116.805 62.9) (end 115.351 62.9) (width 0.8) (layer "F.Cu") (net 6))
 (segment (start 143.3575 67.0175) (end 138.8495 67.0175) (width 0.7) (layer "F.Cu") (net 6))
 (segment (start 136.967 68.9) (end 134.239 68.9) (width 0.7) (layer "F.Cu") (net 6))
 (segment (start 120.5 62.9) (end 118.399 62.9) (width 0.8) (layer "F.Cu") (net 6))
 (segment (start 115.351 62.9) (end 115.316 62.865) (width 0.8) (layer "F.Cu") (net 6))
 (segment (start 118.329 62.9) (end 116.875 62.9) (width 0.8) (layer "F.Cu") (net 6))
 (segment (start 115.281 62.9) (end 113.5 62.9) (width 0.8) (layer "F.Cu") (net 6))
 (segment (start 116.84 62.865) (end 116.805 62.9) (width 0.8) (layer "F.Cu") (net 6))
 (segment (start 125.45 66.35) (end 122.865 66.35) (width 0.7) (layer "F.Cu") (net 6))
 (via (at 116.84 62.865) (size 0.8) (drill 0.4) (layers "F.Cu" "B.Cu") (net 6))
 (via (at 122.428 65.913) (size 0.8) (drill 0.4) (layers "F.Cu" "B.Cu") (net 6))
 (via (at 118.364 62.865) (size 0.8) (drill 0.4) (layers "F.Cu" "B.Cu") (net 6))
 (via (at 115.316 62.865) (size 0.8) (drill 0.4) (layers "F.Cu" "B.Cu") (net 6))
 (segment (start 114.3 65.532) (end 114.3 63.881) (width 0.7) (layer "B.Cu") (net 6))
 (segment (start 114.869 66.101) (end 114.3 65.532) (width 0.7) (layer "B.Cu") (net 6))
 (segment (start 114.3 63.881) (end 115.316 62.865) (width 0.7) (layer "B.Cu") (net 6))
 (segment (start 122.24 66.101) (end 114.869 66.101) (width 0.7) (layer "B.Cu") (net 6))
 (segment (start 122.428 65.913) (end 122.24 66.101) (width 0.7) (layer "B.Cu") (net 6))
 (segment (start 115.316 62.865) (end 118.364 62.865) (width 0.8) (layer "B.Cu") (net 6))
 (segment (start 146.177 61.976) (end 144.2185 60.0175) (width 0.8) (layer "F.Cu") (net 8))
 (segment (start 116.85 67.3) (end 118.354 67.3) (width 0.8) (layer "F.Cu") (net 8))
 (segment (start 116.84 67.31) (end 116.85 67.3) (width 0.8) (layer "F.Cu") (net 8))
 (segment (start 123.05 69.85) (end 144.145 69.85) (width 0.8) (layer "F.Cu") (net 8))
 (segment (start 118.364 67.31) (end 118.374 67.3) (width 0.8) (layer "F.Cu") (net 8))
 (segment (start 115.316 67.31) (end 115.326 67.3) (width 0.8) (layer "F.Cu") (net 8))
 (segment (start 118.354 67.3) (end 118.364 67.31) (width 0.8) (layer "F.Cu") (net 8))
 (segment (start 144.2185 60.0175) (end 143.3575 60.0175) (width 0.8) (layer "F.Cu") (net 8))
 (segment (start 116.83 67.3) (end 116.84 67.31) (width 0.8) (layer "F.Cu") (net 8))
 (segment (start 118.374 67.3) (end 120.5 67.3) (width 0.8) (layer "F.Cu") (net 8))
 (segment (start 120.5 67.3) (end 123.05 69.85) (width 0.8) (layer "F.Cu") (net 8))
 (segment (start 113.5 67.3) (end 115.306 67.3) (width 0.8) (layer "F.Cu") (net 8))
 (segment (start 115.306 67.3) (end 115.316 67.31) (width 0.8) (layer "F.Cu") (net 8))
 (segment (start 144.145 69.85) (end 146.177 67.818) (width 0.8) (layer "F.Cu") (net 8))
 (segment (start 146.177 67.818) (end 146.177 61.976) (width 0.8) (layer "F.Cu") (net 8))
 (segment (start 115.326 67.3) (end 116.83 67.3) (width 0.8) (layer "F.Cu") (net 8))
 (via (at 115.316 67.31) (size 0.8) (drill 0.4) (layers "F.Cu" "B.Cu") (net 8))
 (via (at 116.84 67.31) (size 0.8) (drill 0.4) (layers "F.Cu" "B.Cu") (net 8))
 (via (at 118.364 67.31) (size 0.8) (drill 0.4) (layers "F.Cu" "B.Cu") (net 8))
 (segment (start 121.793 64.008) (end 112.703932 64.008) (width 0.3) (layer "F.Cu") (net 10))
 (segment (start 110.998 65.713932) (end 110.998 66.214) (width 0.3) (layer "F.Cu") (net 10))
 (segment (start 112.703932 64.008) (end 110.998 65.713932) (width 0.3) (layer "F.Cu") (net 10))
 (segment (start 123.063 65.278) (end 121.793 64.008) (width 0.3) (layer "F.Cu") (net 10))
 (segment (start 128.397 65.278) (end 123.063 65.278) (width 0.3) (layer "F.Cu") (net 10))
 (segment (start 130.419 67.3) (end 128.397 65.278) (width 0.3) (layer "F.Cu") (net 10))
 (segment (start 131 67.3) (end 130.419 67.3) (width 0.3) (layer "F.Cu") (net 10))
 (segment (start 112.1075 59.7) (end 110.998 60.8095) (width 0.3) (layer "F.Cu") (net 1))
 (segment (start 113.5 59.7) (end 112.1075 59.7) (width 0.3) (layer "F.Cu") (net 1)))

